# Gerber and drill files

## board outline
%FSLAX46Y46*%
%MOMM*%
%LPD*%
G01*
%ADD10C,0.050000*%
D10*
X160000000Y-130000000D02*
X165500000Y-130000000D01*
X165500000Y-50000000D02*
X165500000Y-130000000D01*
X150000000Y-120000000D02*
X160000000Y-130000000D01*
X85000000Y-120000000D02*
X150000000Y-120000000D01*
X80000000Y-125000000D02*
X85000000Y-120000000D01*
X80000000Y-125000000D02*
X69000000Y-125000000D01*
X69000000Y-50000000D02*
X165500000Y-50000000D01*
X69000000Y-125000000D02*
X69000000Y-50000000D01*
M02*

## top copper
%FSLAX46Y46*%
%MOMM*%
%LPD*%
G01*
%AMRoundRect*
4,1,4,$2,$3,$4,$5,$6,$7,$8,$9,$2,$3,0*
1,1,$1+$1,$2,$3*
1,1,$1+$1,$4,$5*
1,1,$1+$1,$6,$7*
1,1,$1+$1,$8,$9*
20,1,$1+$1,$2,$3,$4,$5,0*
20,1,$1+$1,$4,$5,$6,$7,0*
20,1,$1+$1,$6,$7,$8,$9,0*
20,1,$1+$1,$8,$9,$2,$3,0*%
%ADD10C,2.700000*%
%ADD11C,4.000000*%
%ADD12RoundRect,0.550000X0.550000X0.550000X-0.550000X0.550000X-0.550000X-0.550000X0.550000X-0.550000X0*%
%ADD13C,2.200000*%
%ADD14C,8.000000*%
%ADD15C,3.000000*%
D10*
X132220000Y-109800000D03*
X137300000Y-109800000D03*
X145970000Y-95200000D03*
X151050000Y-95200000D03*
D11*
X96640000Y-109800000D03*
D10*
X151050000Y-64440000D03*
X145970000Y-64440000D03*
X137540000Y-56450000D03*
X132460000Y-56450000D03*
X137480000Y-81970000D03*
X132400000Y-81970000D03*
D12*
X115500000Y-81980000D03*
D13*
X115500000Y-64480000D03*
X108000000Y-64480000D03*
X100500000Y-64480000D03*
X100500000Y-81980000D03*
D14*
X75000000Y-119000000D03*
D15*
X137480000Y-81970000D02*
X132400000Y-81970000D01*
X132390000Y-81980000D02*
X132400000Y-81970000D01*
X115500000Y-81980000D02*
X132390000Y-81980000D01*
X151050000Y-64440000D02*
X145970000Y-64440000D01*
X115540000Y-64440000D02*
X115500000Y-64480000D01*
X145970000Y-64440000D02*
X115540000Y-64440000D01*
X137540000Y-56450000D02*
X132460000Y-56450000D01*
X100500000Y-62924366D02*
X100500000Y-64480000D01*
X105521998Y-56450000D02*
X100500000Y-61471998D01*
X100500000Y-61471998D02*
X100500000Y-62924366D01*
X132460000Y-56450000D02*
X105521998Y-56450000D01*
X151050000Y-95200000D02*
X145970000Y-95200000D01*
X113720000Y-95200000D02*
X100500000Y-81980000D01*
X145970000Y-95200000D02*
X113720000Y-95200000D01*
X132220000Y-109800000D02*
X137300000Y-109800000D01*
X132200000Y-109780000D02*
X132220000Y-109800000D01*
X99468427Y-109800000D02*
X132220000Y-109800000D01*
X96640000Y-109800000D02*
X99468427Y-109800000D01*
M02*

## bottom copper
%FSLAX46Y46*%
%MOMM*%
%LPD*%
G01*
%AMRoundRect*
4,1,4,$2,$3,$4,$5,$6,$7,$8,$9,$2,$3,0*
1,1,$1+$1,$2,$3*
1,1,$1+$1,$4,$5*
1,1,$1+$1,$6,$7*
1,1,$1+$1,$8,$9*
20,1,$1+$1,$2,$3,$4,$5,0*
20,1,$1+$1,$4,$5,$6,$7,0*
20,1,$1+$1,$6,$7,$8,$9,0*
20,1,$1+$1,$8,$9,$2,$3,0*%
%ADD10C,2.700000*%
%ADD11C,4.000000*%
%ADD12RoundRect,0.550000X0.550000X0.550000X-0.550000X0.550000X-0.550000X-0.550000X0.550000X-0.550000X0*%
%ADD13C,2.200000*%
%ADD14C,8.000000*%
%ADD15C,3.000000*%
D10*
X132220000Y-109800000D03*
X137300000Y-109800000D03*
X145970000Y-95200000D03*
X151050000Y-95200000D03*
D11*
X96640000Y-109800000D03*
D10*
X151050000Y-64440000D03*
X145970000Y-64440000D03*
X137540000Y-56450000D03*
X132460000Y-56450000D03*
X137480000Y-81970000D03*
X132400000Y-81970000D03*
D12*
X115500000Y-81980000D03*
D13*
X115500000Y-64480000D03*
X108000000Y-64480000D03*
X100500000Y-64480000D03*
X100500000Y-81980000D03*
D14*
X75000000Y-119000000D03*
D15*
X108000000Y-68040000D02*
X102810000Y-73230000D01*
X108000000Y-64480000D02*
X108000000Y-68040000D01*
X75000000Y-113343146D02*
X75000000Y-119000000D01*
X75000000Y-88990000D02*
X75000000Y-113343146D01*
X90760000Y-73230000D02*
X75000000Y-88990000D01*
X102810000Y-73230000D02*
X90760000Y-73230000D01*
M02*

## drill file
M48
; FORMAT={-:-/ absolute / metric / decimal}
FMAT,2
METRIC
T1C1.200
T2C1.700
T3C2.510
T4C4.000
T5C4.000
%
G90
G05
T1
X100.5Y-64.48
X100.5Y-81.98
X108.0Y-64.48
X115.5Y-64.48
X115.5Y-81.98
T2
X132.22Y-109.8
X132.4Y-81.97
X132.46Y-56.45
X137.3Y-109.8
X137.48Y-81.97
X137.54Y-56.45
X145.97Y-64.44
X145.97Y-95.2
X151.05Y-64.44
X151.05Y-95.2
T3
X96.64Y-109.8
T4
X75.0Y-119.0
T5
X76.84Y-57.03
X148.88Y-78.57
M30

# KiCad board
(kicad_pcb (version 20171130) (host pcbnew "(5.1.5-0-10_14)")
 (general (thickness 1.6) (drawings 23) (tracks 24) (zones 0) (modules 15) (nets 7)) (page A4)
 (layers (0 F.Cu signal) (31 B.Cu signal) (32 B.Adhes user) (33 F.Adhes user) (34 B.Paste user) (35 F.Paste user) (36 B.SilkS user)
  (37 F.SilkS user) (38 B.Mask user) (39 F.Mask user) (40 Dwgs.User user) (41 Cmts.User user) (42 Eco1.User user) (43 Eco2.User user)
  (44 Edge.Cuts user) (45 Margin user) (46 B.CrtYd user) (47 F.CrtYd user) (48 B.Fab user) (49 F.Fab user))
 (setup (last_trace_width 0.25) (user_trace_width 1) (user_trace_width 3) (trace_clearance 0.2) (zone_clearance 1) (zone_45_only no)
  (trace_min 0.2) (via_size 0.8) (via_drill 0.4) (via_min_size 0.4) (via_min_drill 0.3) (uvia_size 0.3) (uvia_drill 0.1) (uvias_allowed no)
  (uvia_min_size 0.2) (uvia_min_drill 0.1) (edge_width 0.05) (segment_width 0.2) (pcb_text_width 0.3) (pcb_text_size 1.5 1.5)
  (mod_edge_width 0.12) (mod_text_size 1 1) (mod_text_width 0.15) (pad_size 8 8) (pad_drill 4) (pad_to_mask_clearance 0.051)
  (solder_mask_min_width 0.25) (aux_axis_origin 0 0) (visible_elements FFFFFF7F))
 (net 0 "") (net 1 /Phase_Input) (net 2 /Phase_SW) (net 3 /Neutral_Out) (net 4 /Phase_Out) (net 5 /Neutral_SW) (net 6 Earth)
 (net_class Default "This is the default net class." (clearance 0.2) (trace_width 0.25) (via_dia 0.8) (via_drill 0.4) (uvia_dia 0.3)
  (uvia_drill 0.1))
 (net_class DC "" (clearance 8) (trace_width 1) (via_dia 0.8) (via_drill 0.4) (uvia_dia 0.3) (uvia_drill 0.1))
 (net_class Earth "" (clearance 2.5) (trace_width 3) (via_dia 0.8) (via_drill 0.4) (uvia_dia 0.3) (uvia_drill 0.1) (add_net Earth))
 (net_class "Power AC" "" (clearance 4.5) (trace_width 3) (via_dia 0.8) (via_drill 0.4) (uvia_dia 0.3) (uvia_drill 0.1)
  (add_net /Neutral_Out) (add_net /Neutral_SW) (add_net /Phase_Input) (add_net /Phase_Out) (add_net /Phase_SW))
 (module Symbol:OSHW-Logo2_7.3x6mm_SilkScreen (layer F.Cu) (at 161.46 106.13 90)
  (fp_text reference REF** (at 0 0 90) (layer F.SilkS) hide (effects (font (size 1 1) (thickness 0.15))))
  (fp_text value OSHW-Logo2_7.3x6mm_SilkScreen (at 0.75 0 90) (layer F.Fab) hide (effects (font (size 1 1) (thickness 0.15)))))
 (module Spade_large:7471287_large (layer F.Cu) (at 132.22 109.8)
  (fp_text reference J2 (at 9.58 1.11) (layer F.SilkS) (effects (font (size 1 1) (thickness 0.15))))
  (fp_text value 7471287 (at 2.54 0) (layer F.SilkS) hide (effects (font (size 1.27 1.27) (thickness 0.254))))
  (pad 1 thru_hole circle (at 0 0) (size 2.7 2.7) (drill 1.7) (layers *.Cu *.Mask) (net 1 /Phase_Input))
  (pad 2 thru_hole circle (at 5.08 0) (size 2.7 2.7) (drill 1.7) (layers *.Cu *.Mask) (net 1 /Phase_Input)))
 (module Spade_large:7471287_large (layer F.Cu) (at 151.05 95.2 180)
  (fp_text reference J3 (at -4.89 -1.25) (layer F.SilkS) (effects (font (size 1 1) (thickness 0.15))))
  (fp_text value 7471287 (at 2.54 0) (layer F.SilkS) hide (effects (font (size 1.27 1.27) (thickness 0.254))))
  (pad 2 thru_hole circle (at 5.08 0 180) (size 2.7 2.7) (drill 1.7) (layers *.Cu *.Mask) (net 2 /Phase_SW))
  (pad 1 thru_hole circle (at 0 0 180) (size 2.7 2.7) (drill 1.7) (layers *.Cu *.Mask) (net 2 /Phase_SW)))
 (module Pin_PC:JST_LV (layer F.Cu) (at 96.64 109.8 180)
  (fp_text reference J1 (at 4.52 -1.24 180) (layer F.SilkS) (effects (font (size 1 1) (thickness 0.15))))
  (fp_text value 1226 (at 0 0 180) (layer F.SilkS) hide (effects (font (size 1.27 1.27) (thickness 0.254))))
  (pad 1 thru_hole circle (at 0 0 270) (size 4 4) (drill 2.51) (layers *.Cu *.Mask F.SilkS) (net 1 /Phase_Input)))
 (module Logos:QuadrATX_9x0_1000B (layer F.Cu) (at 88.71 86.58 90)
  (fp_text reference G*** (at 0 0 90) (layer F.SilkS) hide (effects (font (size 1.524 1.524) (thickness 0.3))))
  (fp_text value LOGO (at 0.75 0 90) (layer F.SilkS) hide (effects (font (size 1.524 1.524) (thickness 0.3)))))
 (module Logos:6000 (layer F.Cu) (at 77.03 86.32)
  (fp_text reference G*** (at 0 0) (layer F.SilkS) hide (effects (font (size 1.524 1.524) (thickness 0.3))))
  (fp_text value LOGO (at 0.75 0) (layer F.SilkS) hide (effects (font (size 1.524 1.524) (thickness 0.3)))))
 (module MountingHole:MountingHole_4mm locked (layer F.Cu) (at 76.84 57.03)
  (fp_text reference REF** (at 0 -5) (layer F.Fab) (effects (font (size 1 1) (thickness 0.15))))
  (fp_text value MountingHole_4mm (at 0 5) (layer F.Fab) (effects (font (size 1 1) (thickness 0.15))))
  (pad 1 np_thru_hole circle (at 0 0) (size 4 4) (drill 4) (layers *.Cu *.Mask)))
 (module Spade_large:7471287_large (layer F.Cu) (at 145.97 64.44)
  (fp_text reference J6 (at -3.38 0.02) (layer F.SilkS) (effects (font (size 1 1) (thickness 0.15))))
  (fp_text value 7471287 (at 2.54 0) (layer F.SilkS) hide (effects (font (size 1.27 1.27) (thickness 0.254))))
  (pad 2 thru_hole circle (at 5.08 0) (size 2.7 2.7) (drill 1.7) (layers *.Cu *.Mask) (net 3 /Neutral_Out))
  (pad 1 thru_hole circle (at 0 0) (size 2.7 2.7) (drill 1.7) (layers *.Cu *.Mask) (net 3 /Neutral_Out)))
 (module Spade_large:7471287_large (layer F.Cu) (at 132.46 56.45)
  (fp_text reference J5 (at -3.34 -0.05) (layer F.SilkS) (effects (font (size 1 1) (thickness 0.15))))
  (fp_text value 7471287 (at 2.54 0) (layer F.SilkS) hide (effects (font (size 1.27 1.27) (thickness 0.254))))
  (pad 2 thru_hole circle (at 5.08 0) (size 2.7 2.7) (drill 1.7) (layers *.Cu *.Mask) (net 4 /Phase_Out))
  (pad 1 thru_hole circle (at 0 0) (size 2.7 2.7) (drill 1.7) (layers *.Cu *.Mask) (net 4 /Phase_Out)))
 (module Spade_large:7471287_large (layer F.Cu) (at 132.4 81.97)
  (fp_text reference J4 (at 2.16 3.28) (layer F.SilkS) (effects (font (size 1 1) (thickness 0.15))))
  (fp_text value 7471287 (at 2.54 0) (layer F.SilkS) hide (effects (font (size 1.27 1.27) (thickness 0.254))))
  (pad 2 thru_hole circle (at 5.08 0) (size 2.7 2.7) (drill 1.7) (layers *.Cu *.Mask) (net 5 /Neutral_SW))
  (pad 1 thru_hole circle (at 0 0) (size 2.7 2.7) (drill 1.7) (layers *.Cu *.Mask) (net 5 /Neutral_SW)))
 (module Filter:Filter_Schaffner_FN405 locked (layer F.Cu) (at 115.5 81.98 180)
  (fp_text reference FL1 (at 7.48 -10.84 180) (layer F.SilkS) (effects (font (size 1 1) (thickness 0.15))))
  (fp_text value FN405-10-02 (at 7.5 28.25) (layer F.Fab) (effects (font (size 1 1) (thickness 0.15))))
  (pad 1 thru_hole roundrect (at 0 0 180) (size 2.2 2.2) (drill 1.2) (layers *.Cu *.Mask) (roundrect_rratio 0.25) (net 5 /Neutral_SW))
  (pad 2 thru_hole circle (at 0 17.5 180) (size 2.2 2.2) (drill 1.2) (layers *.Cu *.Mask) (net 3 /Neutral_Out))
  (pad 3 thru_hole circle (at 7.5 17.5 180) (size 2.2 2.2) (drill 1.2) (layers *.Cu *.Mask) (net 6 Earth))
  (pad 4 thru_hole circle (at 15 17.5 180) (size 2.2 2.2) (drill 1.2) (layers *.Cu *.Mask) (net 4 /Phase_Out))
  (pad 5 thru_hole circle (at 15 0 180) (size 2.2 2.2) (drill 1.2) (layers *.Cu *.Mask) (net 2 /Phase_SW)))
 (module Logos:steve (layer F.Cu) (at 161.04 123.37 90)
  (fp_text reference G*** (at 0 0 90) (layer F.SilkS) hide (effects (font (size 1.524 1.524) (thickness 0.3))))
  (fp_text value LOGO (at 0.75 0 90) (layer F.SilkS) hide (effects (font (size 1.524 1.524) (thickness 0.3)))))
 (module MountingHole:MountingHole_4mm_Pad (layer F.Cu) (at 75 119)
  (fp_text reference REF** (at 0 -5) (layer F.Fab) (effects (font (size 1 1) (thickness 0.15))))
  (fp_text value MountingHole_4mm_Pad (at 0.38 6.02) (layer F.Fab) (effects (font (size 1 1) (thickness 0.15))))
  (pad 1 thru_hole circle (at 0 0) (size 8 8) (drill 4) (layers *.Cu *.Mask) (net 6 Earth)))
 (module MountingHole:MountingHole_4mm (layer F.Cu) (at 148.88 78.57)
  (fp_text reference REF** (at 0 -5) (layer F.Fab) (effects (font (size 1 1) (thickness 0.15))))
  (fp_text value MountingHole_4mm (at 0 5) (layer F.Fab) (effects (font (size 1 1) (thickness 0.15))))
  (pad 1 np_thru_hole circle (at 0 0) (size 4 4) (drill 4) (layers *.Cu *.Mask)))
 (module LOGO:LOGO (layer F.Cu) (at 81.25 72.5)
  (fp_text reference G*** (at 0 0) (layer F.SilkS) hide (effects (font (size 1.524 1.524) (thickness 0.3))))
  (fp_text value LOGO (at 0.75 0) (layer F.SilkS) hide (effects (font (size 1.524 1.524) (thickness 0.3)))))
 (gr_line (start 160 130) (end 165.5 130) (layer Edge.Cuts) (width 0.05))
 (gr_line (start 165.5 50) (end 165.5 130) (layer Edge.Cuts) (width 0.05))
 (gr_line (start 150 120) (end 160 130) (layer Edge.Cuts) (width 0.05))
 (gr_line (start 85 120) (end 150 120) (layer Edge.Cuts) (width 0.05))
 (gr_line (start 80 125) (end 85 120) (layer Edge.Cuts) (width 0.05))
 (gr_line (start 80 125) (end 69 125) (layer Edge.Cuts) (width 0.05))
 (gr_line (start 69 50) (end 165.5 50) (layer Edge.Cuts) (width 0.05))
 (gr_line (start 69 125) (end 69 50) (layer Edge.Cuts) (width 0.05))
 (segment (start 108 68.04) (end 102.81 73.23) (width 3) (layer B.Cu) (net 6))
 (segment (start 108 64.48) (end 108 68.04) (width 3) (layer B.Cu) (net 6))
 (segment (start 75 113.343146) (end 75 119) (width 3) (layer B.Cu) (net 6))
 (segment (start 75 88.99) (end 75 113.343146) (width 3) (layer B.Cu) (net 6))
 (segment (start 90.76 73.23) (end 75 88.99) (width 3) (layer B.Cu) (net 6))
 (segment (start 102.81 73.23) (end 90.76 73.23) (width 3) (layer B.Cu) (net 6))
 (segment (start 137.48 81.97) (end 132.4 81.97) (width 3) (layer F.Cu) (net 5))
 (segment (start 132.39 81.98) (end 132.4 81.97) (width 3) (layer F.Cu) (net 5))
 (segment (start 115.5 81.98) (end 132.39 81.98) (width 3) (layer F.Cu) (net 5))
 (segment (start 151.05 64.44) (end 145.97 64.44) (width 3) (layer F.Cu) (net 3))
 (segment (start 115.54 64.44) (end 115.5 64.48) (width 3) (layer F.Cu) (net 3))
 (segment (start 145.97 64.44) (end 115.54 64.44) (width 3) (layer F.Cu) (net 3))
 (segment (start 137.54 56.45) (end 132.46 56.45) (width 3) (layer F.Cu) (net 4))
 (segment (start 100.5 62.924366) (end 100.5 64.48) (width 3) (layer F.Cu) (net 4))
 (segment (start 105.521998 56.45) (end 100.5 61.471998) (width 3) (layer F.Cu) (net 4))
 (segment (start 100.5 61.471998) (end 100.5 62.924366) (width 3) (layer F.Cu) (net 4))
 (segment (start 132.46 56.45) (end 105.521998 56.45) (width 3) (layer F.Cu) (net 4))
 (segment (start 151.05 95.2) (end 145.97 95.2) (width 3) (layer F.Cu) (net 2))
 (segment (start 113.72 95.2) (end 100.5 81.98) (width 3) (layer F.Cu) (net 2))
 (segment (start 145.97 95.2) (end 113.72 95.2) (width 3) (layer F.Cu) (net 2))
 (segment (start 132.22 109.8) (end 137.3 109.8) (width 3) (layer F.Cu) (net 1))
 (segment (start 132.2 109.78) (end 132.22 109.8) (width 3) (layer F.Cu) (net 1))
 (segment (start 99.468427 109.8) (end 132.22 109.8) (width 3) (layer F.Cu) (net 1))
 (segment (start 96.64 109.8) (end 99.468427 109.8) (width 3) (layer F.Cu) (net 1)))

